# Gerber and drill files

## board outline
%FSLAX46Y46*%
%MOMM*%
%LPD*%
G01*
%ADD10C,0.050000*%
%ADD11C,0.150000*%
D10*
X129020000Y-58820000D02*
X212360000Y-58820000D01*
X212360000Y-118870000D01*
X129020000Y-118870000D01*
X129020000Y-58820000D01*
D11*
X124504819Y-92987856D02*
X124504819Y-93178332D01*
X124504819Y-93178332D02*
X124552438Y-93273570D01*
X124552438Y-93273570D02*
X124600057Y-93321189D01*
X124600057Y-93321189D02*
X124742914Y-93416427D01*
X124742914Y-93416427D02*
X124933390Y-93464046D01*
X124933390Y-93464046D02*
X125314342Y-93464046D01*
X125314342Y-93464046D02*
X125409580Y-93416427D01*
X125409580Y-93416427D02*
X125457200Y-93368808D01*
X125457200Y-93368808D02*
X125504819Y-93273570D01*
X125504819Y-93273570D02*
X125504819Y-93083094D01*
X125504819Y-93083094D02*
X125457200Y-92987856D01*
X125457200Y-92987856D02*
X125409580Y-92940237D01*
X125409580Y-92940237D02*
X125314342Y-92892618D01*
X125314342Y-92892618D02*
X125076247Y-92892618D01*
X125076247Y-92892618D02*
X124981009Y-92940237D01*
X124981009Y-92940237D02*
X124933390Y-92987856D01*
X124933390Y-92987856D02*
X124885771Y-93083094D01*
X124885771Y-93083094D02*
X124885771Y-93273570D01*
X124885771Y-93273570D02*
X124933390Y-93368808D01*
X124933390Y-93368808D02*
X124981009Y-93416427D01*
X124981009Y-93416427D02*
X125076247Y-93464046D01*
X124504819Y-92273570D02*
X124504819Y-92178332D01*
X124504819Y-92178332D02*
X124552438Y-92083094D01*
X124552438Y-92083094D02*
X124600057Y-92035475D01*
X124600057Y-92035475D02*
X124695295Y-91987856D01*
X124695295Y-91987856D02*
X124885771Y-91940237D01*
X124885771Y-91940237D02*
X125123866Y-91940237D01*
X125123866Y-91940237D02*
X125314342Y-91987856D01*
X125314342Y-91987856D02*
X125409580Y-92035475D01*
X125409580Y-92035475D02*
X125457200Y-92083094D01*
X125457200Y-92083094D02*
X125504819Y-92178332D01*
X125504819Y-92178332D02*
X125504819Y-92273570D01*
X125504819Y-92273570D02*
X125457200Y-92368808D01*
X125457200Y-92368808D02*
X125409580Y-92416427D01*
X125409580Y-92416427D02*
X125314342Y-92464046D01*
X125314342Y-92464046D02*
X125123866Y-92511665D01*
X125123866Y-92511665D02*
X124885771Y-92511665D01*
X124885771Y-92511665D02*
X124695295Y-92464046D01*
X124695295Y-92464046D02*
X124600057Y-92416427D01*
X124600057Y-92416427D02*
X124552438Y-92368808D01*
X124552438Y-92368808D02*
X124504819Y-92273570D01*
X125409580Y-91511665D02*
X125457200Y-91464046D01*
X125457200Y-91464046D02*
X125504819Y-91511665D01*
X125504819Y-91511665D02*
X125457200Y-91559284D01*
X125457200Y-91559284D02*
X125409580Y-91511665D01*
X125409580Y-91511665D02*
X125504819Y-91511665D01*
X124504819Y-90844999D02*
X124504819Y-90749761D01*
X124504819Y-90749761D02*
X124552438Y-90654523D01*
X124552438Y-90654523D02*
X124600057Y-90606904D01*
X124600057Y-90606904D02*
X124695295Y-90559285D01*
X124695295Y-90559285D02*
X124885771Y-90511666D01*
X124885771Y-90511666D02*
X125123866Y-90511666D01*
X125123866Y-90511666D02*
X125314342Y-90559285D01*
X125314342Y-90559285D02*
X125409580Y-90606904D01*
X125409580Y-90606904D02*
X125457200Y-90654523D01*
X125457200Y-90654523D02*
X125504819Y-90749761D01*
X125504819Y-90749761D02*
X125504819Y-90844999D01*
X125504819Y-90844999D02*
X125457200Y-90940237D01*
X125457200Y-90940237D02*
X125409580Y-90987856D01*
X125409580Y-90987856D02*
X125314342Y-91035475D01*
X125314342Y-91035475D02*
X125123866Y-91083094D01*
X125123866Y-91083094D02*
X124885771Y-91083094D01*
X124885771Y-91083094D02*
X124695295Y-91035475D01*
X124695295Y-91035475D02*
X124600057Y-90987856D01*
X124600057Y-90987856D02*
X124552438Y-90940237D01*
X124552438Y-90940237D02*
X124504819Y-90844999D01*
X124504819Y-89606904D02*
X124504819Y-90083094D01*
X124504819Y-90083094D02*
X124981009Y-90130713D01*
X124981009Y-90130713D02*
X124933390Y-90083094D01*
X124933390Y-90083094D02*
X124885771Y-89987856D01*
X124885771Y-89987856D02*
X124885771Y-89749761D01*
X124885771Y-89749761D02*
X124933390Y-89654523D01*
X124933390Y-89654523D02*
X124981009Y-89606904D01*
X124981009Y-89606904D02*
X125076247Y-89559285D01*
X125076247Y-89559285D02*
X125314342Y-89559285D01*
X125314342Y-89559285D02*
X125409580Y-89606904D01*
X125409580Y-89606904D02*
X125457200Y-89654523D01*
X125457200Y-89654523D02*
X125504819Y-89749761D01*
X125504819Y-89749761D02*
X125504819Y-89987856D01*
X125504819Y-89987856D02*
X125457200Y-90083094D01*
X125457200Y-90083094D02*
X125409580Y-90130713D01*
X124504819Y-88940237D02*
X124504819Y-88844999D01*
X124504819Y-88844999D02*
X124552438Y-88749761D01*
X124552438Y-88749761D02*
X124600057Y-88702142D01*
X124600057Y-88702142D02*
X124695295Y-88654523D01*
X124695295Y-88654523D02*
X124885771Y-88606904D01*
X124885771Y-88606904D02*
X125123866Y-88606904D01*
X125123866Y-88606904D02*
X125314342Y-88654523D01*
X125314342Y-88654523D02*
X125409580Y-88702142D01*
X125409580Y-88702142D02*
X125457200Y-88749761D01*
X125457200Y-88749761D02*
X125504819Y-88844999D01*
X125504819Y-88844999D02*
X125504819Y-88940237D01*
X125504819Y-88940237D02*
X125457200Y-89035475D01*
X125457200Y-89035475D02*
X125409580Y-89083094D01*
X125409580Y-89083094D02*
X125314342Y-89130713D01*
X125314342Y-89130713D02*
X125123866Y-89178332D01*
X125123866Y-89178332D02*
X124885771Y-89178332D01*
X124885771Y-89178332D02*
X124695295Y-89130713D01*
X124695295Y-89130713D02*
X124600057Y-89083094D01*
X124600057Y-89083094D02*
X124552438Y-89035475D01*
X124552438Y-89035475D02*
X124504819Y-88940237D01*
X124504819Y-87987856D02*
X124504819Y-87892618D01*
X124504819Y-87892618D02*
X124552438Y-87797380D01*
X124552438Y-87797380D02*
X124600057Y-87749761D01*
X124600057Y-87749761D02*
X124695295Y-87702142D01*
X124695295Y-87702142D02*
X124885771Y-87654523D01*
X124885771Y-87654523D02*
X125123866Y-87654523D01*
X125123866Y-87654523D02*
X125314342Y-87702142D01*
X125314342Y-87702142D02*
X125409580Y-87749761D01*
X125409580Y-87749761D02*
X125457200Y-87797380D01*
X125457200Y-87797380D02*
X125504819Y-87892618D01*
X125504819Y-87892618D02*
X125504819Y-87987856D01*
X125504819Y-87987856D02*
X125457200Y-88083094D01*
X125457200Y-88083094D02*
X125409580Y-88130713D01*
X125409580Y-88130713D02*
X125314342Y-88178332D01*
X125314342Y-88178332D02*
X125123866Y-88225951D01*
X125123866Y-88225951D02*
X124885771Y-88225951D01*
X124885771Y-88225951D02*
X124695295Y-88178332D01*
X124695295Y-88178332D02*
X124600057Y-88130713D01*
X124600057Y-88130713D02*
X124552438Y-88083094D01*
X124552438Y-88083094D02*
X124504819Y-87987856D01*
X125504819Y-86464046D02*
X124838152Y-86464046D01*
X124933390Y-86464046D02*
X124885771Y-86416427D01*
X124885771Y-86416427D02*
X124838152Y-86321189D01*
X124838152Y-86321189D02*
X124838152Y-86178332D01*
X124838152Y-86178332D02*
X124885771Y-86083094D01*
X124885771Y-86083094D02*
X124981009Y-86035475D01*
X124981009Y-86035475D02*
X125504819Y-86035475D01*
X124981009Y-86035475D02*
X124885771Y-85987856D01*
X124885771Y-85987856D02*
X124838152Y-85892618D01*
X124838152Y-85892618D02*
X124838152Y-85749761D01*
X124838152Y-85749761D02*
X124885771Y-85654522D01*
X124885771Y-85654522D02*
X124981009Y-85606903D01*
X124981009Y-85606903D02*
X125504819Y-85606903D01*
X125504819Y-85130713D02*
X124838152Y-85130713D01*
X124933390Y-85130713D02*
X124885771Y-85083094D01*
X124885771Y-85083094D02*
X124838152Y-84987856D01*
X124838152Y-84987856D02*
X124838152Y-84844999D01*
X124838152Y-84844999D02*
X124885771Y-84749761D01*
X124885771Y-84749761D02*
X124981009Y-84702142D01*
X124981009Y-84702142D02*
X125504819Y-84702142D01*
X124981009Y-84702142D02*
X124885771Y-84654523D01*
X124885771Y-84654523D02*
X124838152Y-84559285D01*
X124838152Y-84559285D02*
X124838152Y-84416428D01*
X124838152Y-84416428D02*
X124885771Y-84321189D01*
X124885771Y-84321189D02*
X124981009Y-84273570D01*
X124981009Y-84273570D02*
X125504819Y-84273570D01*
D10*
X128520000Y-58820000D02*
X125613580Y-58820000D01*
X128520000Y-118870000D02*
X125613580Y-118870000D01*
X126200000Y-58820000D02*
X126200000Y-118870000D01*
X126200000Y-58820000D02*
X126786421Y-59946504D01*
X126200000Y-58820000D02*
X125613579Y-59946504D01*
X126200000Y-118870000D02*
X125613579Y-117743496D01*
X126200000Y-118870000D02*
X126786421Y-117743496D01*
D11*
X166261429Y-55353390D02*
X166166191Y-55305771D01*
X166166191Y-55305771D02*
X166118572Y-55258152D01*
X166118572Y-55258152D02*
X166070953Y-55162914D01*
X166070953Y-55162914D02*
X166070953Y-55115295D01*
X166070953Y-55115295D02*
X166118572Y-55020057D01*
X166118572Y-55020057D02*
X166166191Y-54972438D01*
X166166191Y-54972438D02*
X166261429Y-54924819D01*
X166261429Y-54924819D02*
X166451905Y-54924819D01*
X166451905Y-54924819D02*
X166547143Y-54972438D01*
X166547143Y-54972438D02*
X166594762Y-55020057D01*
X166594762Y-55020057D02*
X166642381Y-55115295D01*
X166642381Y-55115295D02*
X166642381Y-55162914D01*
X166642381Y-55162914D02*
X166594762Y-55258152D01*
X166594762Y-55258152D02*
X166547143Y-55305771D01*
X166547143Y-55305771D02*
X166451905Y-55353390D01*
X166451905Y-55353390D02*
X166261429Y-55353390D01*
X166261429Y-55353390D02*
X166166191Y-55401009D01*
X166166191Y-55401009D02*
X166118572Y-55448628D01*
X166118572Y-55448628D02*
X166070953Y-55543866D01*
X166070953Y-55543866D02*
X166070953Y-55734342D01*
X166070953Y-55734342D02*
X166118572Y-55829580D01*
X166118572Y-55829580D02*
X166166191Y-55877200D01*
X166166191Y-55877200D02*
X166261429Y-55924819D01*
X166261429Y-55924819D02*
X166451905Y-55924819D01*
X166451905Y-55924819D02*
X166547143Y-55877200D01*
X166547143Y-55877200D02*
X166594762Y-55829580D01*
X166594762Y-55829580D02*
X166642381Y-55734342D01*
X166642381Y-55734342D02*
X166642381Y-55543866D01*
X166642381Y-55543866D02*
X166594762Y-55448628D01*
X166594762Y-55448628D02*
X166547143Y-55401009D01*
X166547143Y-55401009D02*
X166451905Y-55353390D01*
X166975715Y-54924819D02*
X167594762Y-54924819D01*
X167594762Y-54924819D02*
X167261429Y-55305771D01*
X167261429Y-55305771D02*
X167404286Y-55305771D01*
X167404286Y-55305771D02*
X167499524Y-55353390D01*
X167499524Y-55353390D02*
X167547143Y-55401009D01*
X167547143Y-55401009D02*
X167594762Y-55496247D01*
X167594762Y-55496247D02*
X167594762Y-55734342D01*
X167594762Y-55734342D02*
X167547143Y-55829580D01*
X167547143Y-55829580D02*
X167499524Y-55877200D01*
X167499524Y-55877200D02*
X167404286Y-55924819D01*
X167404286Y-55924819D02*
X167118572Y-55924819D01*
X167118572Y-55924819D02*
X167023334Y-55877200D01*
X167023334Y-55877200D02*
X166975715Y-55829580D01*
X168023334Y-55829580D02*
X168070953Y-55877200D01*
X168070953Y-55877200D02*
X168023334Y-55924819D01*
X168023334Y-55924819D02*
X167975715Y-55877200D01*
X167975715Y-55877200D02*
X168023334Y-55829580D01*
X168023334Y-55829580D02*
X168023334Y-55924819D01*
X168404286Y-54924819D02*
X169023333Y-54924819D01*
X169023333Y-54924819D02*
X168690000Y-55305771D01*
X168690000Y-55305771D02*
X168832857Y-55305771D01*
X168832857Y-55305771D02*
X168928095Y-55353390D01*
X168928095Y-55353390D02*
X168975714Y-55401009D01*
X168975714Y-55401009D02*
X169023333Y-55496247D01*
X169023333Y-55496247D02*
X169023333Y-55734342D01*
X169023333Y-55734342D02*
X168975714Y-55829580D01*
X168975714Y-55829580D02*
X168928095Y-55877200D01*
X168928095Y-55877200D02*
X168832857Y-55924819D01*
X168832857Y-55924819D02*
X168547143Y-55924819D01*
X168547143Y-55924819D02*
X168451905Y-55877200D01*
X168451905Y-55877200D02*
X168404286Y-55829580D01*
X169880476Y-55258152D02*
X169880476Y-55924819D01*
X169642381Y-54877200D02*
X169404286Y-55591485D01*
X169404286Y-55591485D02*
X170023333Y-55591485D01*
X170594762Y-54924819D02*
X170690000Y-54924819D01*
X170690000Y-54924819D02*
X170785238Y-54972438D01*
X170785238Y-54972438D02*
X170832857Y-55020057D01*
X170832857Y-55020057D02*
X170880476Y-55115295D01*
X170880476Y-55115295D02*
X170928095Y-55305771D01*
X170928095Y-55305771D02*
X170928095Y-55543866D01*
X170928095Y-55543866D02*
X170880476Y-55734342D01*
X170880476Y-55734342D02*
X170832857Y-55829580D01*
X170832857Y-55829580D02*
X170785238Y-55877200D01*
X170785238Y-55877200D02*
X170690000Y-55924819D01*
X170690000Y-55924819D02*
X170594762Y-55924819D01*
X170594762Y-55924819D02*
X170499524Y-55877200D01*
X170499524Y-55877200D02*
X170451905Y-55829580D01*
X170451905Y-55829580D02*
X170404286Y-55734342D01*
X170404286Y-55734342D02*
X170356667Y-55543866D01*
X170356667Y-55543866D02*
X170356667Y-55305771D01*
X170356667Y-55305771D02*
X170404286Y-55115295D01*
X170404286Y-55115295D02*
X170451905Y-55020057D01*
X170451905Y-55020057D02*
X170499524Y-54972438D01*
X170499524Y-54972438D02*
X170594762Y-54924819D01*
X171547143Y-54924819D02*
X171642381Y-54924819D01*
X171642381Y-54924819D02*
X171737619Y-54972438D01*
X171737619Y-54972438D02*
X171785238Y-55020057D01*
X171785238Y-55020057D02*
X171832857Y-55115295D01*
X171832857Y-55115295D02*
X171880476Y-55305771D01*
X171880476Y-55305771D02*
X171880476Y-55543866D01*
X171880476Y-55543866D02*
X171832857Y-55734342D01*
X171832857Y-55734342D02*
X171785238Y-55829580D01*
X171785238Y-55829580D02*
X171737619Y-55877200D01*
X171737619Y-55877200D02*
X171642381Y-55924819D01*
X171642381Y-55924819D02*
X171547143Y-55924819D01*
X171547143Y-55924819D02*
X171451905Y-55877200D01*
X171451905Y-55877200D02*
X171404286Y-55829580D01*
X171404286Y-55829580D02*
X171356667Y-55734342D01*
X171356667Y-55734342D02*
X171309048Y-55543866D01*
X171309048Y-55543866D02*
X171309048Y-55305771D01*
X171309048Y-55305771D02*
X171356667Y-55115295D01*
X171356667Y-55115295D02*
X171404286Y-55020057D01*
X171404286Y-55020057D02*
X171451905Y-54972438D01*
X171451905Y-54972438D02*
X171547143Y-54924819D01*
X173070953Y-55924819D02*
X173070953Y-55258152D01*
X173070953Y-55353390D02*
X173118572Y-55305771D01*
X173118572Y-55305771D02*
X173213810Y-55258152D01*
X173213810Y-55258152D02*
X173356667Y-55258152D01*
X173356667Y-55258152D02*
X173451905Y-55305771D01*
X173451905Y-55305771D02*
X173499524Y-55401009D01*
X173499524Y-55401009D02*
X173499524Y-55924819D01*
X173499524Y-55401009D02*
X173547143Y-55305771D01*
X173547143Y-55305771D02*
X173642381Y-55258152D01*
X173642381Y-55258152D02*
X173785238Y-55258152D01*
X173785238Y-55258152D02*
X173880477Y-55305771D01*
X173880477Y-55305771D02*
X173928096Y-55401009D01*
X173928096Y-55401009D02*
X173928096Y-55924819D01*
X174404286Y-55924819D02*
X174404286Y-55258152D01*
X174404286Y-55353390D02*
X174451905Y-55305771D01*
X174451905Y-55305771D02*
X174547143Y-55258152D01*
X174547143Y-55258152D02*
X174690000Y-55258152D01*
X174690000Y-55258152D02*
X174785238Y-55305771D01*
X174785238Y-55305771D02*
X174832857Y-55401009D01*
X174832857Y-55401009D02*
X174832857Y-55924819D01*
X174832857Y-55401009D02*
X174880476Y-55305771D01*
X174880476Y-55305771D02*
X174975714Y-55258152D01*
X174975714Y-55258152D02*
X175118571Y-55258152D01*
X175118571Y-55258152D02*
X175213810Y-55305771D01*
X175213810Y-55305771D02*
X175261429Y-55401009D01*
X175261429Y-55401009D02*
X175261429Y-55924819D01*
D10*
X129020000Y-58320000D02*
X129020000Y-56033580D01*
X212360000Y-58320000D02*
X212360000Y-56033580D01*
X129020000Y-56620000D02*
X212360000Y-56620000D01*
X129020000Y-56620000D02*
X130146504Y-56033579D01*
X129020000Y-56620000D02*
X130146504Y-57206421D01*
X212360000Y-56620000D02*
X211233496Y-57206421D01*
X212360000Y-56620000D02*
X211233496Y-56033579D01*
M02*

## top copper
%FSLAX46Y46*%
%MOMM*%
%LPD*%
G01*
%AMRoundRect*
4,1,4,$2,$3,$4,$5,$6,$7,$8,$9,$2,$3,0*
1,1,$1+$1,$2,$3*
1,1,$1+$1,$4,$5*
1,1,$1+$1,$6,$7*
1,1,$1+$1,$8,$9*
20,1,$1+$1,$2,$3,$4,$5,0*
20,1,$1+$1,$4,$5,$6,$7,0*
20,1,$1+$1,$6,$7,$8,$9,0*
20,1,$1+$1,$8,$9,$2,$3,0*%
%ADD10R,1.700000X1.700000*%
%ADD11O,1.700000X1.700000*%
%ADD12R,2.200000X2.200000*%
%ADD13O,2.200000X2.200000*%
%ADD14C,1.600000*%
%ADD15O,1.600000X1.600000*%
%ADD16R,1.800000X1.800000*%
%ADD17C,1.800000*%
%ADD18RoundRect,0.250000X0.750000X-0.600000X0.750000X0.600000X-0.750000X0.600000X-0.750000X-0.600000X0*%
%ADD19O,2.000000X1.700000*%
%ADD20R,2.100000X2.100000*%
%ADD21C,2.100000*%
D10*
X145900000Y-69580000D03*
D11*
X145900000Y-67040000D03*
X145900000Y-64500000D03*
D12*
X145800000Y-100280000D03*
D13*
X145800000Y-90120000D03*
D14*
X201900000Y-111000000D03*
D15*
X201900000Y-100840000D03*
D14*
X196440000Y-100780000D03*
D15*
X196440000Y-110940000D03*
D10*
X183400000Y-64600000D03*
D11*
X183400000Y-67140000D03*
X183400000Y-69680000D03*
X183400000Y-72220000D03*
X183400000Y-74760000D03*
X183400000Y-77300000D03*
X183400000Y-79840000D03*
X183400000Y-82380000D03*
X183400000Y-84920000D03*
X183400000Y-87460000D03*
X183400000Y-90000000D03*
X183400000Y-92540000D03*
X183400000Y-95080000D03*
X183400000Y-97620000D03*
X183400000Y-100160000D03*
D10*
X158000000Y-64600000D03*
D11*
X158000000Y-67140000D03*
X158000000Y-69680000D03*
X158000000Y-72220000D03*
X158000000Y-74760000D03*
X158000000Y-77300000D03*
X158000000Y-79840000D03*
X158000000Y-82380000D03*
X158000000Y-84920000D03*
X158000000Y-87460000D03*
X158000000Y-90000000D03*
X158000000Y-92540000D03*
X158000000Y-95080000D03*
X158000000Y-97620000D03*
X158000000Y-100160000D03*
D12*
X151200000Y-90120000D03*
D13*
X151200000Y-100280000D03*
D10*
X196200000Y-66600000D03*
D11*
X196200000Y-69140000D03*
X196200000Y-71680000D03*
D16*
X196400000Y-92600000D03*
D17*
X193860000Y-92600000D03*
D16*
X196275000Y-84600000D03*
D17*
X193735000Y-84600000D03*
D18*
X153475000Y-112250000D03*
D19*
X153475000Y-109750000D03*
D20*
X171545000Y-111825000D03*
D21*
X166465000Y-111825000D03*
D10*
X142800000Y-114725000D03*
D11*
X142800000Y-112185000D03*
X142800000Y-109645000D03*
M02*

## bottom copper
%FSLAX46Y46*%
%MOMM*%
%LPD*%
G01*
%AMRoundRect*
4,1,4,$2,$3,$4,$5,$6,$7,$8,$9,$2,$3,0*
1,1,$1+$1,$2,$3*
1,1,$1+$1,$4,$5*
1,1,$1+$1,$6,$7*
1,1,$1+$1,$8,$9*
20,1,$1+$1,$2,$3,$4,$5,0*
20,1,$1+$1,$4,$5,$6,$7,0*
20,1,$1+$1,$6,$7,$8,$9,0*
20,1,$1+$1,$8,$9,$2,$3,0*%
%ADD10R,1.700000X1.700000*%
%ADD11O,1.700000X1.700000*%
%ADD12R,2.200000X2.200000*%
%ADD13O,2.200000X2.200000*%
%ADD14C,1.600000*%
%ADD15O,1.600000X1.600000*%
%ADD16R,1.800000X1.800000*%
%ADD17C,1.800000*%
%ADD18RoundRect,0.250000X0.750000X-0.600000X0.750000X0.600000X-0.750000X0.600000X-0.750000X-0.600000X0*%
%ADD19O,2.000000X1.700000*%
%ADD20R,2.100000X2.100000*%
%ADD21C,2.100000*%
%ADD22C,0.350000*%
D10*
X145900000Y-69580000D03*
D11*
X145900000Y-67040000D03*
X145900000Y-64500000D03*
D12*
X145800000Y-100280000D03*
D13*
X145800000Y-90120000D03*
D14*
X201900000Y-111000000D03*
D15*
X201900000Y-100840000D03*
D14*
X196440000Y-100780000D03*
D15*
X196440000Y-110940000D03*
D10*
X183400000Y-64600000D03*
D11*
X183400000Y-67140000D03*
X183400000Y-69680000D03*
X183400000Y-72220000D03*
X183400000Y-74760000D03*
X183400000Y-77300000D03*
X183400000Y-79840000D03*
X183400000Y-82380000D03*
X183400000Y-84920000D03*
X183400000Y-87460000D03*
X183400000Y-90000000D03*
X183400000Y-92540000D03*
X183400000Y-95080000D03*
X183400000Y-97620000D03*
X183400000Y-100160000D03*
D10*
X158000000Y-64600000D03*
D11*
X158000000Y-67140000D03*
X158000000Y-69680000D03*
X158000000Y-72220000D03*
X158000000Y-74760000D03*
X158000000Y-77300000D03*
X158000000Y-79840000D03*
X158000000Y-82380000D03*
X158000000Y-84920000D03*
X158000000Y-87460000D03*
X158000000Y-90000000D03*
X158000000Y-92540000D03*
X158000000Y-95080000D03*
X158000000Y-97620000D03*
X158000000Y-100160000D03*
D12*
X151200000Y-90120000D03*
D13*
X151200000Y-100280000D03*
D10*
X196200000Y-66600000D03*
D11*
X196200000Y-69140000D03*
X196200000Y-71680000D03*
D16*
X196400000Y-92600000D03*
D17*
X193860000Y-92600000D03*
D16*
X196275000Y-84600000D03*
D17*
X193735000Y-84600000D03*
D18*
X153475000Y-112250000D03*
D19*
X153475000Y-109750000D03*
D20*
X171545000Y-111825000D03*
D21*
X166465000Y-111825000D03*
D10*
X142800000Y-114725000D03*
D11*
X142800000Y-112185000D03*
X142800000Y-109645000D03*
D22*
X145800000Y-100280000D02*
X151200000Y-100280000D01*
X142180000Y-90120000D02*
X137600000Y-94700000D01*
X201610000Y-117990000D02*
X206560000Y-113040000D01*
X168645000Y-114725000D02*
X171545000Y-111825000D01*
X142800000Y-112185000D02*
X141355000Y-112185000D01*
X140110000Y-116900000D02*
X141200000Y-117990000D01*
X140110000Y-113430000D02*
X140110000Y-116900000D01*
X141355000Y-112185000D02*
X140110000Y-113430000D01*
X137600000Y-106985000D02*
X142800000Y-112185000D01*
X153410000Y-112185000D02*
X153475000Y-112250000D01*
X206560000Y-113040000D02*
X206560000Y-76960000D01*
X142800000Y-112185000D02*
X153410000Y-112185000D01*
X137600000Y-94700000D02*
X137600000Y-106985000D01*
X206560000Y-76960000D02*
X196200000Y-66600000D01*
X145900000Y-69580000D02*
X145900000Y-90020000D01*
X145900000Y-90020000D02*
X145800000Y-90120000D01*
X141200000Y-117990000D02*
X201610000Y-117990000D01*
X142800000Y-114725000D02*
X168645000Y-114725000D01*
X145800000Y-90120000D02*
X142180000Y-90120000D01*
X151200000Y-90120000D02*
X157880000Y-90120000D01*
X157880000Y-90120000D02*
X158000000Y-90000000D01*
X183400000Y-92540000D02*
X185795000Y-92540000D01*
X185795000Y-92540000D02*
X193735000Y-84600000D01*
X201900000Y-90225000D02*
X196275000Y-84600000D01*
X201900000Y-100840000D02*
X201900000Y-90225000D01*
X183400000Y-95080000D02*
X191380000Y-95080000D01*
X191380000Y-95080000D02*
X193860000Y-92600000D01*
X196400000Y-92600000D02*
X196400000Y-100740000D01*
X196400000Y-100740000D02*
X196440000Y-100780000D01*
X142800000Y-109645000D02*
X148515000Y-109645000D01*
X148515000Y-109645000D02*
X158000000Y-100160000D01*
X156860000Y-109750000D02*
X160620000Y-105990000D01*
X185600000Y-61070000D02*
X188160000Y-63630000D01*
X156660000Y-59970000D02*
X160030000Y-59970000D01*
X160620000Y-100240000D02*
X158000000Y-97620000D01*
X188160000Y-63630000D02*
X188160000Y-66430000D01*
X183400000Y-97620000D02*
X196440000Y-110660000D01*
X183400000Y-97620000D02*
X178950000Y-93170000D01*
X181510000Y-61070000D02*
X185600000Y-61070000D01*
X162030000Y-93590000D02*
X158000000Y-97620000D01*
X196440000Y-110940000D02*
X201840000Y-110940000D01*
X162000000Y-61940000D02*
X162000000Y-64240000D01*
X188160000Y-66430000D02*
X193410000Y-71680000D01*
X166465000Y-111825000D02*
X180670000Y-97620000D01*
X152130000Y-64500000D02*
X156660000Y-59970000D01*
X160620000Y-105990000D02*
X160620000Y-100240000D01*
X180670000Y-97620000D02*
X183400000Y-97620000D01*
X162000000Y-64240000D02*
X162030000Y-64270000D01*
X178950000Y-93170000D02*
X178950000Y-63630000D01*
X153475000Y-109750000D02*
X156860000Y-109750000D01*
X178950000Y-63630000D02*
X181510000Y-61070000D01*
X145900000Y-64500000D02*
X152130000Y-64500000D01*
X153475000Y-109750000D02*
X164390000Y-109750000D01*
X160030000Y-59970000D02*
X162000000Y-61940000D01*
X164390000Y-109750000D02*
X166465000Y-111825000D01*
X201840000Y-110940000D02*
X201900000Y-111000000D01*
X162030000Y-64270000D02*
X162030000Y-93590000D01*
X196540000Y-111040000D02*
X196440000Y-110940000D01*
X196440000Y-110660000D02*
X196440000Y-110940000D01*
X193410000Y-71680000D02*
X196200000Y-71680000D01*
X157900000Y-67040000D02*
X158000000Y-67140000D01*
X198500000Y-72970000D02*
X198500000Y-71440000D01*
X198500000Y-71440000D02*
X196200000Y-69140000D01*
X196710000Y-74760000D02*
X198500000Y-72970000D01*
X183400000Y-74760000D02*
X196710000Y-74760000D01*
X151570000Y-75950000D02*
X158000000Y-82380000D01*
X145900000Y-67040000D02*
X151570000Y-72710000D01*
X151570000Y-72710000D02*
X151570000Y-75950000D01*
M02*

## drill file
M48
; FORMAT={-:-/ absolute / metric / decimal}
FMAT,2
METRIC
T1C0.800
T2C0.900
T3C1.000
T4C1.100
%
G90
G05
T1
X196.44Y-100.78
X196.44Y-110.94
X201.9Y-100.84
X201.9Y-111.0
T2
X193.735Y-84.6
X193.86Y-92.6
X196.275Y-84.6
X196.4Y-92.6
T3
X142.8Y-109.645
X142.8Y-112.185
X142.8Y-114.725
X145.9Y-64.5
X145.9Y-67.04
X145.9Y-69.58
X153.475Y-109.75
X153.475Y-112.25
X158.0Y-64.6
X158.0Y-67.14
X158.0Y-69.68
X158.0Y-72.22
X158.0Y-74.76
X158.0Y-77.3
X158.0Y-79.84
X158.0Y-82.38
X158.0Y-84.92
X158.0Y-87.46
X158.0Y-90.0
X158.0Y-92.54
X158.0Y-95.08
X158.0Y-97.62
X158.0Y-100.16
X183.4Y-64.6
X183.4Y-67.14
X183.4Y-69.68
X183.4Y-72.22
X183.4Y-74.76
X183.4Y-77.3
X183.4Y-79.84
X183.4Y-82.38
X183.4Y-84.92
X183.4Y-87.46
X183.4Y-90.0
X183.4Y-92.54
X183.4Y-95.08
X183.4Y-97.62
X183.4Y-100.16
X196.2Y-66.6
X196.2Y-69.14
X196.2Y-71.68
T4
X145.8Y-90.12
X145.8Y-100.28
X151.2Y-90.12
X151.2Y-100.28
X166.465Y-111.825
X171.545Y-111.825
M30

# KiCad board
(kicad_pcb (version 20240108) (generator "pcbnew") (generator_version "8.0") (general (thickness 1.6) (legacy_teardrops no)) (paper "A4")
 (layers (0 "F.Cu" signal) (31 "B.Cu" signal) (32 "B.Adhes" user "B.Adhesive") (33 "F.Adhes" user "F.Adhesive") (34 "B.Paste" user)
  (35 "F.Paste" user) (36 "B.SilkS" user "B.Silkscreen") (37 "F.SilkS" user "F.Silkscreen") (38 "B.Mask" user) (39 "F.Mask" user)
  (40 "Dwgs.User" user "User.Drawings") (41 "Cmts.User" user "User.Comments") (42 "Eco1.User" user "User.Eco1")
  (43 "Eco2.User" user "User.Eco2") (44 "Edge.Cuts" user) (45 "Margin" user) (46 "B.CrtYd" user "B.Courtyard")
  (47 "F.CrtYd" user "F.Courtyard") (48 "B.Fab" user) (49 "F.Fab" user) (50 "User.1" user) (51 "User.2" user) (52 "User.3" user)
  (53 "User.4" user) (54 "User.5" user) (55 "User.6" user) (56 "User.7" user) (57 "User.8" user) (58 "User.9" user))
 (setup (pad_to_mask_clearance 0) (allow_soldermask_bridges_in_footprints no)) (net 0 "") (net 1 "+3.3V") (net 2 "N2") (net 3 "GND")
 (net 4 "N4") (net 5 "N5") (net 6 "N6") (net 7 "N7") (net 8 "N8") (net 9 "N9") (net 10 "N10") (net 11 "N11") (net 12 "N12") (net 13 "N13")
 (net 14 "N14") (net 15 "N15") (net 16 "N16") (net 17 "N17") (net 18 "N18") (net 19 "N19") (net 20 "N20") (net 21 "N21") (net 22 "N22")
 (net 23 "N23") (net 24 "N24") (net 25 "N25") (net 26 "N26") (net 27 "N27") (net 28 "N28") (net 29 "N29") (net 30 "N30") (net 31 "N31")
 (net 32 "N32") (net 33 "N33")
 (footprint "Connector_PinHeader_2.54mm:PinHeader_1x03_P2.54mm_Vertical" (layer "F.Cu") (at 145.9 69.58 180)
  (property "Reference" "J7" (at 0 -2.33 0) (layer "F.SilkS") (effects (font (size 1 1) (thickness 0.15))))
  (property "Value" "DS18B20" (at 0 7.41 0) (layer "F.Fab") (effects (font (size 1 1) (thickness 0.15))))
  (pad "1" thru_hole rect (at 0 0 180) (size 1.7 1.7) (drill 1) (layers "*.Cu" "*.Mask") (remove_unused_layers no) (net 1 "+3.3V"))
  (pad "2" thru_hole oval (at 0 2.54 180) (size 1.7 1.7) (drill 1) (layers "*.Cu" "*.Mask") (remove_unused_layers no) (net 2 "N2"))
  (pad "3" thru_hole oval (at 0 5.08 180) (size 1.7 1.7) (drill 1) (layers "*.Cu" "*.Mask") (remove_unused_layers no) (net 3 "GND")))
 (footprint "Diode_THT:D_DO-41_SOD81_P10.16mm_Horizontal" (layer "F.Cu") (at 145.8 100.28 90)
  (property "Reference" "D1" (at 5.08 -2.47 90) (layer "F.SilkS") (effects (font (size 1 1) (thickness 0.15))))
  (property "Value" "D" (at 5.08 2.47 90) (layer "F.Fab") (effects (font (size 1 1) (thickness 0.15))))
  (pad "1" thru_hole rect (at 0 0 90) (size 2.2 2.2) (drill 1.1) (layers "*.Cu" "*.Mask") (remove_unused_layers no) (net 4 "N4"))
  (pad "2" thru_hole oval (at 10.16 0 90) (size 2.2 2.2) (drill 1.1) (layers "*.Cu" "*.Mask") (remove_unused_layers no) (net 1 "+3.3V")))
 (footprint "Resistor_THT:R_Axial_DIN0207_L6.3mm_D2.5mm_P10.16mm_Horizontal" (layer "F.Cu") (at 201.9 111 90)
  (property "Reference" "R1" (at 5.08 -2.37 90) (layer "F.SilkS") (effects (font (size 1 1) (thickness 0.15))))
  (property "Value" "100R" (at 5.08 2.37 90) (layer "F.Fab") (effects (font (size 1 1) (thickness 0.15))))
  (pad "1" thru_hole circle (at 0 0 90) (size 1.6 1.6) (drill 0.8) (layers "*.Cu" "*.Mask") (remove_unused_layers no) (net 3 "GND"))
  (pad "2" thru_hole oval (at 10.16 0 90) (size 1.6 1.6) (drill 0.8) (layers "*.Cu" "*.Mask") (remove_unused_layers no) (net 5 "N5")))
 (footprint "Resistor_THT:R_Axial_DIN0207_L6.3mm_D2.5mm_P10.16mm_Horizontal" (layer "F.Cu") (at 196.44 100.78 -90)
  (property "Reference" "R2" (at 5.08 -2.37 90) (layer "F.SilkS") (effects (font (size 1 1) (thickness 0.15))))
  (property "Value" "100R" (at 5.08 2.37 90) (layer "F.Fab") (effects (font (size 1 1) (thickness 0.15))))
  (pad "1" thru_hole circle (at 0 0 270) (size 1.6 1.6) (drill 0.8) (layers "*.Cu" "*.Mask") (remove_unused_layers no) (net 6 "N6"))
  (pad "2" thru_hole oval (at 10.16 0 270) (size 1.6 1.6) (drill 0.8) (layers "*.Cu" "*.Mask") (remove_unused_layers no) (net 3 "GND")))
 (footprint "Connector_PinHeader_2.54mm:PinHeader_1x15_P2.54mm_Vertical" (layer "F.Cu") (at 183.4 64.6)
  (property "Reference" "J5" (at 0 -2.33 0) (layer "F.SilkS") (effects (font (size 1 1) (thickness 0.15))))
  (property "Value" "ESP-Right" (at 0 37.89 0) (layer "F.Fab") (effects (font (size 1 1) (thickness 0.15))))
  (pad "1" thru_hole rect (at 0 0) (size 1.7 1.7) (drill 1) (layers "*.Cu" "*.Mask") (remove_unused_layers no) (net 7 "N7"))
  (pad "2" thru_hole oval (at 0 2.54) (size 1.7 1.7) (drill 1) (layers "*.Cu" "*.Mask") (remove_unused_layers no) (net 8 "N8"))
  (pad "3" thru_hole oval (at 0 5.08) (size 1.7 1.7) (drill 1) (layers "*.Cu" "*.Mask") (remove_unused_layers no) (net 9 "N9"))
  (pad "4" thru_hole oval (at 0 7.62) (size 1.7 1.7) (drill 1) (layers "*.Cu" "*.Mask") (remove_unused_layers no) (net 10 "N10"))
  (pad "5" thru_hole oval (at 0 10.16) (size 1.7 1.7) (drill 1) (layers "*.Cu" "*.Mask") (remove_unused_layers no) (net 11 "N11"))
  (pad "6" thru_hole oval (at 0 12.7) (size 1.7 1.7) (drill 1) (layers "*.Cu" "*.Mask") (remove_unused_layers no) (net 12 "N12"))
  (pad "7" thru_hole oval (at 0 15.24) (size 1.7 1.7) (drill 1) (layers "*.Cu" "*.Mask") (remove_unused_layers no) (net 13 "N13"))
  (pad "8" thru_hole oval (at 0 17.78) (size 1.7 1.7) (drill 1) (layers "*.Cu" "*.Mask") (remove_unused_layers no) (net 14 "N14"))
  (pad "9" thru_hole oval (at 0 20.32) (size 1.7 1.7) (drill 1) (layers "*.Cu" "*.Mask") (remove_unused_layers no) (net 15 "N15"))
  (pad "10" thru_hole oval (at 0 22.86) (size 1.7 1.7) (drill 1) (layers "*.Cu" "*.Mask") (remove_unused_layers no) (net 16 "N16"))
  (pad "11" thru_hole oval (at 0 25.4) (size 1.7 1.7) (drill 1) (layers "*.Cu" "*.Mask") (remove_unused_layers no) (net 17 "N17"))
  (pad "12" thru_hole oval (at 0 27.94) (size 1.7 1.7) (drill 1) (layers "*.Cu" "*.Mask") (remove_unused_layers no) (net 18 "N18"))
  (pad "13" thru_hole oval (at 0 30.48) (size 1.7 1.7) (drill 1) (layers "*.Cu" "*.Mask") (remove_unused_layers no) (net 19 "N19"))
  (pad "14" thru_hole oval (at 0 33.02) (size 1.7 1.7) (drill 1) (layers "*.Cu" "*.Mask") (remove_unused_layers no) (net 3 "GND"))
  (pad "15" thru_hole oval (at 0 35.56) (size 1.7 1.7) (drill 1) (layers "*.Cu" "*.Mask") (remove_unused_layers no) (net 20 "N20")))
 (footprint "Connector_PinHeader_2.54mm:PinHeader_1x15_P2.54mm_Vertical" (layer "F.Cu") (at 158 64.6)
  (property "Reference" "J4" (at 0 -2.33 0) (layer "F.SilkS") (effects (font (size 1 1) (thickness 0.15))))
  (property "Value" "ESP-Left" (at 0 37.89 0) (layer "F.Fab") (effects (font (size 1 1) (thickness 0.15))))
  (pad "1" thru_hole rect (at 0 0) (size 1.7 1.7) (drill 1) (layers "*.Cu" "*.Mask") (remove_unused_layers no) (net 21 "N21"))
  (pad "2" thru_hole oval (at 0 2.54) (size 1.7 1.7) (drill 1) (layers "*.Cu" "*.Mask") (remove_unused_layers no) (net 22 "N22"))
  (pad "3" thru_hole oval (at 0 5.08) (size 1.7 1.7) (drill 1) (layers "*.Cu" "*.Mask") (remove_unused_layers no) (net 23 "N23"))
  (pad "4" thru_hole oval (at 0 7.62) (size 1.7 1.7) (drill 1) (layers "*.Cu" "*.Mask") (remove_unused_layers no) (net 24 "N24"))
  (pad "5" thru_hole oval (at 0 10.16) (size 1.7 1.7) (drill 1) (layers "*.Cu" "*.Mask") (remove_unused_layers no) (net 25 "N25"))
  (pad "6" thru_hole oval (at 0 12.7) (size 1.7 1.7) (drill 1) (layers "*.Cu" "*.Mask") (remove_unused_layers no) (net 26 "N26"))
  (pad "7" thru_hole oval (at 0 15.24) (size 1.7 1.7) (drill 1) (layers "*.Cu" "*.Mask") (remove_unused_layers no) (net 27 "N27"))
  (pad "8" thru_hole oval (at 0 17.78) (size 1.7 1.7) (drill 1) (layers "*.Cu" "*.Mask") (remove_unused_layers no) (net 2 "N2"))
  (pad "9" thru_hole oval (at 0 20.32) (size 1.7 1.7) (drill 1) (layers "*.Cu" "*.Mask") (remove_unused_layers no) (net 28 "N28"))
  (pad "10" thru_hole oval (at 0 22.86) (size 1.7 1.7) (drill 1) (layers "*.Cu" "*.Mask") (remove_unused_layers no) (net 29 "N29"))
  (pad "11" thru_hole oval (at 0 25.4) (size 1.7 1.7) (drill 1) (layers "*.Cu" "*.Mask") (remove_unused_layers no) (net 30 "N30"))
  (pad "12" thru_hole oval (at 0 27.94) (size 1.7 1.7) (drill 1) (layers "*.Cu" "*.Mask") (remove_unused_layers no) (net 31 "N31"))
  (pad "13" thru_hole oval (at 0 30.48) (size 1.7 1.7) (drill 1) (layers "*.Cu" "*.Mask") (remove_unused_layers no) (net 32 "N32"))
  (pad "14" thru_hole oval (at 0 33.02) (size 1.7 1.7) (drill 1) (layers "*.Cu" "*.Mask") (remove_unused_layers no) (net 3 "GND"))
  (pad "15" thru_hole oval (at 0 35.56) (size 1.7 1.7) (drill 1) (layers "*.Cu" "*.Mask") (remove_unused_layers no) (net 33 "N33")))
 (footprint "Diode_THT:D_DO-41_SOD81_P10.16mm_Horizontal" (layer "F.Cu") (at 151.2 90.12 -90)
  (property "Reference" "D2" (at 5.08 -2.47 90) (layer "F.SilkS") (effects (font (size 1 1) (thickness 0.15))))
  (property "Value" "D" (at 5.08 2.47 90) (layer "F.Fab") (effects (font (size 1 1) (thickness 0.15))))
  (pad "1" thru_hole rect (at 0 0 270) (size 2.2 2.2) (drill 1.1) (layers "*.Cu" "*.Mask") (remove_unused_layers no) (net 30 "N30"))
  (pad "2" thru_hole oval (at 10.16 0 270) (size 2.2 2.2) (drill 1.1) (layers "*.Cu" "*.Mask") (remove_unused_layers no) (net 4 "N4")))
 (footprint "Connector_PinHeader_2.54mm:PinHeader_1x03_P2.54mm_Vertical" (layer "F.Cu") (at 196.2 66.6)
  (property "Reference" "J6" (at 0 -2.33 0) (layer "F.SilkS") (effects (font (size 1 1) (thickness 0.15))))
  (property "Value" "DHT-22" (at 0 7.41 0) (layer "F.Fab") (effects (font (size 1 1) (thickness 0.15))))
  (pad "1" thru_hole rect (at 0 0) (size 1.7 1.7) (drill 1) (layers "*.Cu" "*.Mask") (remove_unused_layers no) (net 1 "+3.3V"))
  (pad "2" thru_hole oval (at 0 2.54) (size 1.7 1.7) (drill 1) (layers "*.Cu" "*.Mask") (remove_unused_layers no) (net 11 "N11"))
  (pad "3" thru_hole oval (at 0 5.08) (size 1.7 1.7) (drill 1) (layers "*.Cu" "*.Mask") (remove_unused_layers no) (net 3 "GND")))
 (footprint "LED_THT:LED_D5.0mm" (layer "F.Cu") (at 196.4 92.6 180)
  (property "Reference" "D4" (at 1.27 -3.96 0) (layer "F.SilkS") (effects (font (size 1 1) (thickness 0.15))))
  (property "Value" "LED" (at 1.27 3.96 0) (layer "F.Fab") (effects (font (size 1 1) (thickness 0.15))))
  (pad "1" thru_hole rect (at 0 0 180) (size 1.8 1.8) (drill 0.9) (layers "*.Cu" "*.Mask") (remove_unused_layers no) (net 6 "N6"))
  (pad "2" thru_hole circle (at 2.54 0 180) (size 1.8 1.8) (drill 0.9) (layers "*.Cu" "*.Mask") (remove_unused_layers no) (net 19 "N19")))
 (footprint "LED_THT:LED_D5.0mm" (layer "F.Cu") (at 196.275 84.6 180)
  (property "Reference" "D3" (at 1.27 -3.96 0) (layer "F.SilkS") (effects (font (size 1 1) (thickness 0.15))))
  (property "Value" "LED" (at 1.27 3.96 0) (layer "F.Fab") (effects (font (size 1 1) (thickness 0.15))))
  (pad "1" thru_hole rect (at 0 0 180) (size 1.8 1.8) (drill 0.9) (layers "*.Cu" "*.Mask") (remove_unused_layers no) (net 5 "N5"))
  (pad "2" thru_hole circle (at 2.54 0 180) (size 1.8 1.8) (drill 0.9) (layers "*.Cu" "*.Mask") (remove_unused_layers no) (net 18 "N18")))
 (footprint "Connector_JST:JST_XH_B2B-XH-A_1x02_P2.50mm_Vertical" (layer "F.Cu") (at 153.475 112.25 90)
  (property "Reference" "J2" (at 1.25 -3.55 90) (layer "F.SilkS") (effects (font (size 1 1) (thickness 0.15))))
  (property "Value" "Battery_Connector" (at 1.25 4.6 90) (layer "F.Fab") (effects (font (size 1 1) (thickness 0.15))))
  (pad "1" thru_hole roundrect (at 0 0 90) (size 1.7 2) (drill 1) (layers "*.Cu" "*.Mask") (remove_unused_layers no)
   (roundrect_rratio 0.147059) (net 1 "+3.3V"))
  (pad "2" thru_hole oval (at 2.5 0 90) (size 1.7 2) (drill 1) (layers "*.Cu" "*.Mask") (remove_unused_layers no) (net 3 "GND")))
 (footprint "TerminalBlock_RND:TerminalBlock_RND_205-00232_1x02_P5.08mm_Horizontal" (layer "F.Cu") (at 171.545 111.825 180)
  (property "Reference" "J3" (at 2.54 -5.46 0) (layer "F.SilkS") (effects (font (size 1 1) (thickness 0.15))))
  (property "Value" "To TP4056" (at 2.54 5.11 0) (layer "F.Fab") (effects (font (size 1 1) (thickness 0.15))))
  (pad "1" thru_hole rect (at 0 0 180) (size 2.1 2.1) (drill 1.1) (layers "*.Cu" "*.Mask") (remove_unused_layers no) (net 1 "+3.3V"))
  (pad "2" thru_hole circle (at 5.08 0 180) (size 2.1 2.1) (drill 1.1) (layers "*.Cu" "*.Mask") (remove_unused_layers no) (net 3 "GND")))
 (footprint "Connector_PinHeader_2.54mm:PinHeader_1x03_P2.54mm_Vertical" (layer "F.Cu") (at 142.8 114.725 180)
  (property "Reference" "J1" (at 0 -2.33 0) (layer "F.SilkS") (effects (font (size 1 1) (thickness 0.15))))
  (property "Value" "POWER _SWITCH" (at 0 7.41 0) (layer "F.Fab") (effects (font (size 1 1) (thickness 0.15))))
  (pad "1" thru_hole rect (at 0 0 180) (size 1.7 1.7) (drill 1) (layers "*.Cu" "*.Mask") (remove_unused_layers no) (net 1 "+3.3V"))
  (pad "2" thru_hole oval (at 0 2.54 180) (size 1.7 1.7) (drill 1) (layers "*.Cu" "*.Mask") (remove_unused_layers no) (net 1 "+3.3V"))
  (pad "3" thru_hole oval (at 0 5.08 180) (size 1.7 1.7) (drill 1) (layers "*.Cu" "*.Mask") (remove_unused_layers no) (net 33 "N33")))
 (gr_rect (start 129.02 58.82) (end 212.36 118.87) (stroke (width 0.05) (type default)) (fill none) (layer "Edge.Cuts"))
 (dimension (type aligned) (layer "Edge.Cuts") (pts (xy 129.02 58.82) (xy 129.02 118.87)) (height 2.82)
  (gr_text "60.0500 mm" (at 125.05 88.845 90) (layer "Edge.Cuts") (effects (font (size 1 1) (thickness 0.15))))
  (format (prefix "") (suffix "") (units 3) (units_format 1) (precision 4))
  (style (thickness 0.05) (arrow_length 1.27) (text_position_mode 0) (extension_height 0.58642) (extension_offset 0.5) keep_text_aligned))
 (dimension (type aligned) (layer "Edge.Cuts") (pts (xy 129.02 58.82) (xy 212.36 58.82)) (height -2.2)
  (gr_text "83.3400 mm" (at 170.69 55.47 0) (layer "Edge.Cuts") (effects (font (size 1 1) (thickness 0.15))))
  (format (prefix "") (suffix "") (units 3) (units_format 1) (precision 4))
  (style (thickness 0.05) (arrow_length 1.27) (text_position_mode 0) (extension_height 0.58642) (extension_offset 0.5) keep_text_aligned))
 (segment (start 145.8 100.28) (end 151.2 100.28) (width 0.35) (layer "B.Cu") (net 4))
 (segment (start 142.18 90.12) (end 137.6 94.7) (width 0.35) (layer "B.Cu") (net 1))
 (segment (start 201.61 117.99) (end 206.56 113.04) (width 0.35) (layer "B.Cu") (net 1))
 (segment (start 168.645 114.725) (end 171.545 111.825) (width 0.35) (layer "B.Cu") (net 1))
 (segment (start 142.8 112.185) (end 141.355 112.185) (width 0.35) (layer "B.Cu") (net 1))
 (segment (start 140.11 116.9) (end 141.2 117.99) (width 0.35) (layer "B.Cu") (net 1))
 (segment (start 140.11 113.43) (end 140.11 116.9) (width 0.35) (layer "B.Cu") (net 1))
 (segment (start 141.355 112.185) (end 140.11 113.43) (width 0.35) (layer "B.Cu") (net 1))
 (segment (start 137.6 106.985) (end 142.8 112.185) (width 0.35) (layer "B.Cu") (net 1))
 (segment (start 153.41 112.185) (end 153.475 112.25) (width 0.35) (layer "B.Cu") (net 1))
 (segment (start 206.56 113.04) (end 206.56 76.96) (width 0.35) (layer "B.Cu") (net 1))
 (segment (start 142.8 112.185) (end 153.41 112.185) (width 0.35) (layer "B.Cu") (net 1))
 (segment (start 137.6 94.7) (end 137.6 106.985) (width 0.35) (layer "B.Cu") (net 1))
 (segment (start 206.56 76.96) (end 196.2 66.6) (width 0.35) (layer "B.Cu") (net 1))
 (segment (start 145.9 69.58) (end 145.9 90.02) (width 0.35) (layer "B.Cu") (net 1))
 (segment (start 145.9 90.02) (end 145.8 90.12) (width 0.35) (layer "B.Cu") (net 1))
 (segment (start 141.2 117.99) (end 201.61 117.99) (width 0.35) (layer "B.Cu") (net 1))
 (segment (start 142.8 114.725) (end 168.645 114.725) (width 0.35) (layer "B.Cu") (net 1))
 (segment (start 145.8 90.12) (end 142.18 90.12) (width 0.35) (layer "B.Cu") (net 1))
 (segment (start 151.2 90.12) (end 157.88 90.12) (width 0.35) (layer "B.Cu") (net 30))
 (segment (start 157.88 90.12) (end 158 90) (width 0.35) (layer "B.Cu") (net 30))
 (segment (start 183.4 92.54) (end 185.795 92.54) (width 0.35) (layer "B.Cu") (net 18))
 (segment (start 185.795 92.54) (end 193.735 84.6) (width 0.35) (layer "B.Cu") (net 18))
 (segment (start 201.9 90.225) (end 196.275 84.6) (width 0.35) (layer "B.Cu") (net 5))
 (segment (start 201.9 100.84) (end 201.9 90.225) (width 0.35) (layer "B.Cu") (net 5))
 (segment (start 183.4 95.08) (end 191.38 95.08) (width 0.35) (layer "B.Cu") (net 19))
 (segment (start 191.38 95.08) (end 193.86 92.6) (width 0.35) (layer "B.Cu") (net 19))
 (segment (start 196.4 92.6) (end 196.4 100.74) (width 0.35) (layer "B.Cu") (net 6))
 (segment (start 196.4 100.74) (end 196.44 100.78) (width 0.35) (layer "B.Cu") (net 6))
 (segment (start 142.8 109.645) (end 148.515 109.645) (width 0.35) (layer "B.Cu") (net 33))
 (segment (start 148.515 109.645) (end 158 100.16) (width 0.35) (layer "B.Cu") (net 33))
 (segment (start 156.86 109.75) (end 160.62 105.99) (width 0.35) (layer "B.Cu") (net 3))
 (segment (start 185.6 61.07) (end 188.16 63.63) (width 0.35) (layer "B.Cu") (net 3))
 (segment (start 156.66 59.97) (end 160.03 59.97) (width 0.35) (layer "B.Cu") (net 3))
 (segment (start 160.62 100.24) (end 158 97.62) (width 0.35) (layer "B.Cu") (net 3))
 (segment (start 188.16 63.63) (end 188.16 66.43) (width 0.35) (layer "B.Cu") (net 3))
 (segment (start 183.4 97.62) (end 196.44 110.66) (width 0.35) (layer "B.Cu") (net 3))
 (segment (start 183.4 97.62) (end 178.95 93.17) (width 0.35) (layer "B.Cu") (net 3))
 (segment (start 181.51 61.07) (end 185.6 61.07) (width 0.35) (layer "B.Cu") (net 3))
 (segment (start 162.03 93.59) (end 158 97.62) (width 0.35) (layer "B.Cu") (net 3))
 (segment (start 196.44 110.94) (end 201.84 110.94) (width 0.35) (layer "B.Cu") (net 3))
 (segment (start 162 61.94) (end 162 64.24) (width 0.35) (layer "B.Cu") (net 3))
 (segment (start 188.16 66.43) (end 193.41 71.68) (width 0.35) (layer "B.Cu") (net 3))
 (segment (start 166.465 111.825) (end 180.67 97.62) (width 0.35) (layer "B.Cu") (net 3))
 (segment (start 152.13 64.5) (end 156.66 59.97) (width 0.35) (layer "B.Cu") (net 3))
 (segment (start 160.62 105.99) (end 160.62 100.24) (width 0.35) (layer "B.Cu") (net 3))
 (segment (start 180.67 97.62) (end 183.4 97.62) (width 0.35) (layer "B.Cu") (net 3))
 (segment (start 162 64.24) (end 162.03 64.27) (width 0.35) (layer "B.Cu") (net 3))
 (segment (start 178.95 93.17) (end 178.95 63.63) (width 0.35) (layer "B.Cu") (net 3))
 (segment (start 153.475 109.75) (end 156.86 109.75) (width 0.35) (layer "B.Cu") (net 3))
 (segment (start 178.95 63.63) (end 181.51 61.07) (width 0.35) (layer "B.Cu") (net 3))
 (segment (start 145.9 64.5) (end 152.13 64.5) (width 0.35) (layer "B.Cu") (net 3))
 (segment (start 153.475 109.75) (end 164.39 109.75) (width 0.35) (layer "B.Cu") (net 3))
 (segment (start 160.03 59.97) (end 162 61.94) (width 0.35) (layer "B.Cu") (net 3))
 (segment (start 164.39 109.75) (end 166.465 111.825) (width 0.35) (layer "B.Cu") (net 3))
 (segment (start 201.84 110.94) (end 201.9 111) (width 0.35) (layer "B.Cu") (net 3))
 (segment (start 162.03 64.27) (end 162.03 93.59) (width 0.35) (layer "B.Cu") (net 3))
 (segment (start 196.54 111.04) (end 196.44 110.94) (width 0.35) (layer "B.Cu") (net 3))
 (segment (start 196.44 110.66) (end 196.44 110.94) (width 0.35) (layer "B.Cu") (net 3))
 (segment (start 193.41 71.68) (end 196.2 71.68) (width 0.35) (layer "B.Cu") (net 3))
 (segment (start 157.9 67.04) (end 158 67.14) (width 0.35) (layer "B.Cu") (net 22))
 (segment (start 198.5 72.97) (end 198.5 71.44) (width 0.35) (layer "B.Cu") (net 11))
 (segment (start 198.5 71.44) (end 196.2 69.14) (width 0.35) (layer "B.Cu") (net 11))
 (segment (start 196.71 74.76) (end 198.5 72.97) (width 0.35) (layer "B.Cu") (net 11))
 (segment (start 183.4 74.76) (end 196.71 74.76) (width 0.35) (layer "B.Cu") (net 11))
 (segment (start 151.57 75.95) (end 158 82.38) (width 0.35) (layer "B.Cu") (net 2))
 (segment (start 145.9 67.04) (end 151.57 72.71) (width 0.35) (layer "B.Cu") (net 2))
 (segment (start 151.57 72.71) (end 151.57 75.95) (width 0.35) (layer "B.Cu") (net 2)))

